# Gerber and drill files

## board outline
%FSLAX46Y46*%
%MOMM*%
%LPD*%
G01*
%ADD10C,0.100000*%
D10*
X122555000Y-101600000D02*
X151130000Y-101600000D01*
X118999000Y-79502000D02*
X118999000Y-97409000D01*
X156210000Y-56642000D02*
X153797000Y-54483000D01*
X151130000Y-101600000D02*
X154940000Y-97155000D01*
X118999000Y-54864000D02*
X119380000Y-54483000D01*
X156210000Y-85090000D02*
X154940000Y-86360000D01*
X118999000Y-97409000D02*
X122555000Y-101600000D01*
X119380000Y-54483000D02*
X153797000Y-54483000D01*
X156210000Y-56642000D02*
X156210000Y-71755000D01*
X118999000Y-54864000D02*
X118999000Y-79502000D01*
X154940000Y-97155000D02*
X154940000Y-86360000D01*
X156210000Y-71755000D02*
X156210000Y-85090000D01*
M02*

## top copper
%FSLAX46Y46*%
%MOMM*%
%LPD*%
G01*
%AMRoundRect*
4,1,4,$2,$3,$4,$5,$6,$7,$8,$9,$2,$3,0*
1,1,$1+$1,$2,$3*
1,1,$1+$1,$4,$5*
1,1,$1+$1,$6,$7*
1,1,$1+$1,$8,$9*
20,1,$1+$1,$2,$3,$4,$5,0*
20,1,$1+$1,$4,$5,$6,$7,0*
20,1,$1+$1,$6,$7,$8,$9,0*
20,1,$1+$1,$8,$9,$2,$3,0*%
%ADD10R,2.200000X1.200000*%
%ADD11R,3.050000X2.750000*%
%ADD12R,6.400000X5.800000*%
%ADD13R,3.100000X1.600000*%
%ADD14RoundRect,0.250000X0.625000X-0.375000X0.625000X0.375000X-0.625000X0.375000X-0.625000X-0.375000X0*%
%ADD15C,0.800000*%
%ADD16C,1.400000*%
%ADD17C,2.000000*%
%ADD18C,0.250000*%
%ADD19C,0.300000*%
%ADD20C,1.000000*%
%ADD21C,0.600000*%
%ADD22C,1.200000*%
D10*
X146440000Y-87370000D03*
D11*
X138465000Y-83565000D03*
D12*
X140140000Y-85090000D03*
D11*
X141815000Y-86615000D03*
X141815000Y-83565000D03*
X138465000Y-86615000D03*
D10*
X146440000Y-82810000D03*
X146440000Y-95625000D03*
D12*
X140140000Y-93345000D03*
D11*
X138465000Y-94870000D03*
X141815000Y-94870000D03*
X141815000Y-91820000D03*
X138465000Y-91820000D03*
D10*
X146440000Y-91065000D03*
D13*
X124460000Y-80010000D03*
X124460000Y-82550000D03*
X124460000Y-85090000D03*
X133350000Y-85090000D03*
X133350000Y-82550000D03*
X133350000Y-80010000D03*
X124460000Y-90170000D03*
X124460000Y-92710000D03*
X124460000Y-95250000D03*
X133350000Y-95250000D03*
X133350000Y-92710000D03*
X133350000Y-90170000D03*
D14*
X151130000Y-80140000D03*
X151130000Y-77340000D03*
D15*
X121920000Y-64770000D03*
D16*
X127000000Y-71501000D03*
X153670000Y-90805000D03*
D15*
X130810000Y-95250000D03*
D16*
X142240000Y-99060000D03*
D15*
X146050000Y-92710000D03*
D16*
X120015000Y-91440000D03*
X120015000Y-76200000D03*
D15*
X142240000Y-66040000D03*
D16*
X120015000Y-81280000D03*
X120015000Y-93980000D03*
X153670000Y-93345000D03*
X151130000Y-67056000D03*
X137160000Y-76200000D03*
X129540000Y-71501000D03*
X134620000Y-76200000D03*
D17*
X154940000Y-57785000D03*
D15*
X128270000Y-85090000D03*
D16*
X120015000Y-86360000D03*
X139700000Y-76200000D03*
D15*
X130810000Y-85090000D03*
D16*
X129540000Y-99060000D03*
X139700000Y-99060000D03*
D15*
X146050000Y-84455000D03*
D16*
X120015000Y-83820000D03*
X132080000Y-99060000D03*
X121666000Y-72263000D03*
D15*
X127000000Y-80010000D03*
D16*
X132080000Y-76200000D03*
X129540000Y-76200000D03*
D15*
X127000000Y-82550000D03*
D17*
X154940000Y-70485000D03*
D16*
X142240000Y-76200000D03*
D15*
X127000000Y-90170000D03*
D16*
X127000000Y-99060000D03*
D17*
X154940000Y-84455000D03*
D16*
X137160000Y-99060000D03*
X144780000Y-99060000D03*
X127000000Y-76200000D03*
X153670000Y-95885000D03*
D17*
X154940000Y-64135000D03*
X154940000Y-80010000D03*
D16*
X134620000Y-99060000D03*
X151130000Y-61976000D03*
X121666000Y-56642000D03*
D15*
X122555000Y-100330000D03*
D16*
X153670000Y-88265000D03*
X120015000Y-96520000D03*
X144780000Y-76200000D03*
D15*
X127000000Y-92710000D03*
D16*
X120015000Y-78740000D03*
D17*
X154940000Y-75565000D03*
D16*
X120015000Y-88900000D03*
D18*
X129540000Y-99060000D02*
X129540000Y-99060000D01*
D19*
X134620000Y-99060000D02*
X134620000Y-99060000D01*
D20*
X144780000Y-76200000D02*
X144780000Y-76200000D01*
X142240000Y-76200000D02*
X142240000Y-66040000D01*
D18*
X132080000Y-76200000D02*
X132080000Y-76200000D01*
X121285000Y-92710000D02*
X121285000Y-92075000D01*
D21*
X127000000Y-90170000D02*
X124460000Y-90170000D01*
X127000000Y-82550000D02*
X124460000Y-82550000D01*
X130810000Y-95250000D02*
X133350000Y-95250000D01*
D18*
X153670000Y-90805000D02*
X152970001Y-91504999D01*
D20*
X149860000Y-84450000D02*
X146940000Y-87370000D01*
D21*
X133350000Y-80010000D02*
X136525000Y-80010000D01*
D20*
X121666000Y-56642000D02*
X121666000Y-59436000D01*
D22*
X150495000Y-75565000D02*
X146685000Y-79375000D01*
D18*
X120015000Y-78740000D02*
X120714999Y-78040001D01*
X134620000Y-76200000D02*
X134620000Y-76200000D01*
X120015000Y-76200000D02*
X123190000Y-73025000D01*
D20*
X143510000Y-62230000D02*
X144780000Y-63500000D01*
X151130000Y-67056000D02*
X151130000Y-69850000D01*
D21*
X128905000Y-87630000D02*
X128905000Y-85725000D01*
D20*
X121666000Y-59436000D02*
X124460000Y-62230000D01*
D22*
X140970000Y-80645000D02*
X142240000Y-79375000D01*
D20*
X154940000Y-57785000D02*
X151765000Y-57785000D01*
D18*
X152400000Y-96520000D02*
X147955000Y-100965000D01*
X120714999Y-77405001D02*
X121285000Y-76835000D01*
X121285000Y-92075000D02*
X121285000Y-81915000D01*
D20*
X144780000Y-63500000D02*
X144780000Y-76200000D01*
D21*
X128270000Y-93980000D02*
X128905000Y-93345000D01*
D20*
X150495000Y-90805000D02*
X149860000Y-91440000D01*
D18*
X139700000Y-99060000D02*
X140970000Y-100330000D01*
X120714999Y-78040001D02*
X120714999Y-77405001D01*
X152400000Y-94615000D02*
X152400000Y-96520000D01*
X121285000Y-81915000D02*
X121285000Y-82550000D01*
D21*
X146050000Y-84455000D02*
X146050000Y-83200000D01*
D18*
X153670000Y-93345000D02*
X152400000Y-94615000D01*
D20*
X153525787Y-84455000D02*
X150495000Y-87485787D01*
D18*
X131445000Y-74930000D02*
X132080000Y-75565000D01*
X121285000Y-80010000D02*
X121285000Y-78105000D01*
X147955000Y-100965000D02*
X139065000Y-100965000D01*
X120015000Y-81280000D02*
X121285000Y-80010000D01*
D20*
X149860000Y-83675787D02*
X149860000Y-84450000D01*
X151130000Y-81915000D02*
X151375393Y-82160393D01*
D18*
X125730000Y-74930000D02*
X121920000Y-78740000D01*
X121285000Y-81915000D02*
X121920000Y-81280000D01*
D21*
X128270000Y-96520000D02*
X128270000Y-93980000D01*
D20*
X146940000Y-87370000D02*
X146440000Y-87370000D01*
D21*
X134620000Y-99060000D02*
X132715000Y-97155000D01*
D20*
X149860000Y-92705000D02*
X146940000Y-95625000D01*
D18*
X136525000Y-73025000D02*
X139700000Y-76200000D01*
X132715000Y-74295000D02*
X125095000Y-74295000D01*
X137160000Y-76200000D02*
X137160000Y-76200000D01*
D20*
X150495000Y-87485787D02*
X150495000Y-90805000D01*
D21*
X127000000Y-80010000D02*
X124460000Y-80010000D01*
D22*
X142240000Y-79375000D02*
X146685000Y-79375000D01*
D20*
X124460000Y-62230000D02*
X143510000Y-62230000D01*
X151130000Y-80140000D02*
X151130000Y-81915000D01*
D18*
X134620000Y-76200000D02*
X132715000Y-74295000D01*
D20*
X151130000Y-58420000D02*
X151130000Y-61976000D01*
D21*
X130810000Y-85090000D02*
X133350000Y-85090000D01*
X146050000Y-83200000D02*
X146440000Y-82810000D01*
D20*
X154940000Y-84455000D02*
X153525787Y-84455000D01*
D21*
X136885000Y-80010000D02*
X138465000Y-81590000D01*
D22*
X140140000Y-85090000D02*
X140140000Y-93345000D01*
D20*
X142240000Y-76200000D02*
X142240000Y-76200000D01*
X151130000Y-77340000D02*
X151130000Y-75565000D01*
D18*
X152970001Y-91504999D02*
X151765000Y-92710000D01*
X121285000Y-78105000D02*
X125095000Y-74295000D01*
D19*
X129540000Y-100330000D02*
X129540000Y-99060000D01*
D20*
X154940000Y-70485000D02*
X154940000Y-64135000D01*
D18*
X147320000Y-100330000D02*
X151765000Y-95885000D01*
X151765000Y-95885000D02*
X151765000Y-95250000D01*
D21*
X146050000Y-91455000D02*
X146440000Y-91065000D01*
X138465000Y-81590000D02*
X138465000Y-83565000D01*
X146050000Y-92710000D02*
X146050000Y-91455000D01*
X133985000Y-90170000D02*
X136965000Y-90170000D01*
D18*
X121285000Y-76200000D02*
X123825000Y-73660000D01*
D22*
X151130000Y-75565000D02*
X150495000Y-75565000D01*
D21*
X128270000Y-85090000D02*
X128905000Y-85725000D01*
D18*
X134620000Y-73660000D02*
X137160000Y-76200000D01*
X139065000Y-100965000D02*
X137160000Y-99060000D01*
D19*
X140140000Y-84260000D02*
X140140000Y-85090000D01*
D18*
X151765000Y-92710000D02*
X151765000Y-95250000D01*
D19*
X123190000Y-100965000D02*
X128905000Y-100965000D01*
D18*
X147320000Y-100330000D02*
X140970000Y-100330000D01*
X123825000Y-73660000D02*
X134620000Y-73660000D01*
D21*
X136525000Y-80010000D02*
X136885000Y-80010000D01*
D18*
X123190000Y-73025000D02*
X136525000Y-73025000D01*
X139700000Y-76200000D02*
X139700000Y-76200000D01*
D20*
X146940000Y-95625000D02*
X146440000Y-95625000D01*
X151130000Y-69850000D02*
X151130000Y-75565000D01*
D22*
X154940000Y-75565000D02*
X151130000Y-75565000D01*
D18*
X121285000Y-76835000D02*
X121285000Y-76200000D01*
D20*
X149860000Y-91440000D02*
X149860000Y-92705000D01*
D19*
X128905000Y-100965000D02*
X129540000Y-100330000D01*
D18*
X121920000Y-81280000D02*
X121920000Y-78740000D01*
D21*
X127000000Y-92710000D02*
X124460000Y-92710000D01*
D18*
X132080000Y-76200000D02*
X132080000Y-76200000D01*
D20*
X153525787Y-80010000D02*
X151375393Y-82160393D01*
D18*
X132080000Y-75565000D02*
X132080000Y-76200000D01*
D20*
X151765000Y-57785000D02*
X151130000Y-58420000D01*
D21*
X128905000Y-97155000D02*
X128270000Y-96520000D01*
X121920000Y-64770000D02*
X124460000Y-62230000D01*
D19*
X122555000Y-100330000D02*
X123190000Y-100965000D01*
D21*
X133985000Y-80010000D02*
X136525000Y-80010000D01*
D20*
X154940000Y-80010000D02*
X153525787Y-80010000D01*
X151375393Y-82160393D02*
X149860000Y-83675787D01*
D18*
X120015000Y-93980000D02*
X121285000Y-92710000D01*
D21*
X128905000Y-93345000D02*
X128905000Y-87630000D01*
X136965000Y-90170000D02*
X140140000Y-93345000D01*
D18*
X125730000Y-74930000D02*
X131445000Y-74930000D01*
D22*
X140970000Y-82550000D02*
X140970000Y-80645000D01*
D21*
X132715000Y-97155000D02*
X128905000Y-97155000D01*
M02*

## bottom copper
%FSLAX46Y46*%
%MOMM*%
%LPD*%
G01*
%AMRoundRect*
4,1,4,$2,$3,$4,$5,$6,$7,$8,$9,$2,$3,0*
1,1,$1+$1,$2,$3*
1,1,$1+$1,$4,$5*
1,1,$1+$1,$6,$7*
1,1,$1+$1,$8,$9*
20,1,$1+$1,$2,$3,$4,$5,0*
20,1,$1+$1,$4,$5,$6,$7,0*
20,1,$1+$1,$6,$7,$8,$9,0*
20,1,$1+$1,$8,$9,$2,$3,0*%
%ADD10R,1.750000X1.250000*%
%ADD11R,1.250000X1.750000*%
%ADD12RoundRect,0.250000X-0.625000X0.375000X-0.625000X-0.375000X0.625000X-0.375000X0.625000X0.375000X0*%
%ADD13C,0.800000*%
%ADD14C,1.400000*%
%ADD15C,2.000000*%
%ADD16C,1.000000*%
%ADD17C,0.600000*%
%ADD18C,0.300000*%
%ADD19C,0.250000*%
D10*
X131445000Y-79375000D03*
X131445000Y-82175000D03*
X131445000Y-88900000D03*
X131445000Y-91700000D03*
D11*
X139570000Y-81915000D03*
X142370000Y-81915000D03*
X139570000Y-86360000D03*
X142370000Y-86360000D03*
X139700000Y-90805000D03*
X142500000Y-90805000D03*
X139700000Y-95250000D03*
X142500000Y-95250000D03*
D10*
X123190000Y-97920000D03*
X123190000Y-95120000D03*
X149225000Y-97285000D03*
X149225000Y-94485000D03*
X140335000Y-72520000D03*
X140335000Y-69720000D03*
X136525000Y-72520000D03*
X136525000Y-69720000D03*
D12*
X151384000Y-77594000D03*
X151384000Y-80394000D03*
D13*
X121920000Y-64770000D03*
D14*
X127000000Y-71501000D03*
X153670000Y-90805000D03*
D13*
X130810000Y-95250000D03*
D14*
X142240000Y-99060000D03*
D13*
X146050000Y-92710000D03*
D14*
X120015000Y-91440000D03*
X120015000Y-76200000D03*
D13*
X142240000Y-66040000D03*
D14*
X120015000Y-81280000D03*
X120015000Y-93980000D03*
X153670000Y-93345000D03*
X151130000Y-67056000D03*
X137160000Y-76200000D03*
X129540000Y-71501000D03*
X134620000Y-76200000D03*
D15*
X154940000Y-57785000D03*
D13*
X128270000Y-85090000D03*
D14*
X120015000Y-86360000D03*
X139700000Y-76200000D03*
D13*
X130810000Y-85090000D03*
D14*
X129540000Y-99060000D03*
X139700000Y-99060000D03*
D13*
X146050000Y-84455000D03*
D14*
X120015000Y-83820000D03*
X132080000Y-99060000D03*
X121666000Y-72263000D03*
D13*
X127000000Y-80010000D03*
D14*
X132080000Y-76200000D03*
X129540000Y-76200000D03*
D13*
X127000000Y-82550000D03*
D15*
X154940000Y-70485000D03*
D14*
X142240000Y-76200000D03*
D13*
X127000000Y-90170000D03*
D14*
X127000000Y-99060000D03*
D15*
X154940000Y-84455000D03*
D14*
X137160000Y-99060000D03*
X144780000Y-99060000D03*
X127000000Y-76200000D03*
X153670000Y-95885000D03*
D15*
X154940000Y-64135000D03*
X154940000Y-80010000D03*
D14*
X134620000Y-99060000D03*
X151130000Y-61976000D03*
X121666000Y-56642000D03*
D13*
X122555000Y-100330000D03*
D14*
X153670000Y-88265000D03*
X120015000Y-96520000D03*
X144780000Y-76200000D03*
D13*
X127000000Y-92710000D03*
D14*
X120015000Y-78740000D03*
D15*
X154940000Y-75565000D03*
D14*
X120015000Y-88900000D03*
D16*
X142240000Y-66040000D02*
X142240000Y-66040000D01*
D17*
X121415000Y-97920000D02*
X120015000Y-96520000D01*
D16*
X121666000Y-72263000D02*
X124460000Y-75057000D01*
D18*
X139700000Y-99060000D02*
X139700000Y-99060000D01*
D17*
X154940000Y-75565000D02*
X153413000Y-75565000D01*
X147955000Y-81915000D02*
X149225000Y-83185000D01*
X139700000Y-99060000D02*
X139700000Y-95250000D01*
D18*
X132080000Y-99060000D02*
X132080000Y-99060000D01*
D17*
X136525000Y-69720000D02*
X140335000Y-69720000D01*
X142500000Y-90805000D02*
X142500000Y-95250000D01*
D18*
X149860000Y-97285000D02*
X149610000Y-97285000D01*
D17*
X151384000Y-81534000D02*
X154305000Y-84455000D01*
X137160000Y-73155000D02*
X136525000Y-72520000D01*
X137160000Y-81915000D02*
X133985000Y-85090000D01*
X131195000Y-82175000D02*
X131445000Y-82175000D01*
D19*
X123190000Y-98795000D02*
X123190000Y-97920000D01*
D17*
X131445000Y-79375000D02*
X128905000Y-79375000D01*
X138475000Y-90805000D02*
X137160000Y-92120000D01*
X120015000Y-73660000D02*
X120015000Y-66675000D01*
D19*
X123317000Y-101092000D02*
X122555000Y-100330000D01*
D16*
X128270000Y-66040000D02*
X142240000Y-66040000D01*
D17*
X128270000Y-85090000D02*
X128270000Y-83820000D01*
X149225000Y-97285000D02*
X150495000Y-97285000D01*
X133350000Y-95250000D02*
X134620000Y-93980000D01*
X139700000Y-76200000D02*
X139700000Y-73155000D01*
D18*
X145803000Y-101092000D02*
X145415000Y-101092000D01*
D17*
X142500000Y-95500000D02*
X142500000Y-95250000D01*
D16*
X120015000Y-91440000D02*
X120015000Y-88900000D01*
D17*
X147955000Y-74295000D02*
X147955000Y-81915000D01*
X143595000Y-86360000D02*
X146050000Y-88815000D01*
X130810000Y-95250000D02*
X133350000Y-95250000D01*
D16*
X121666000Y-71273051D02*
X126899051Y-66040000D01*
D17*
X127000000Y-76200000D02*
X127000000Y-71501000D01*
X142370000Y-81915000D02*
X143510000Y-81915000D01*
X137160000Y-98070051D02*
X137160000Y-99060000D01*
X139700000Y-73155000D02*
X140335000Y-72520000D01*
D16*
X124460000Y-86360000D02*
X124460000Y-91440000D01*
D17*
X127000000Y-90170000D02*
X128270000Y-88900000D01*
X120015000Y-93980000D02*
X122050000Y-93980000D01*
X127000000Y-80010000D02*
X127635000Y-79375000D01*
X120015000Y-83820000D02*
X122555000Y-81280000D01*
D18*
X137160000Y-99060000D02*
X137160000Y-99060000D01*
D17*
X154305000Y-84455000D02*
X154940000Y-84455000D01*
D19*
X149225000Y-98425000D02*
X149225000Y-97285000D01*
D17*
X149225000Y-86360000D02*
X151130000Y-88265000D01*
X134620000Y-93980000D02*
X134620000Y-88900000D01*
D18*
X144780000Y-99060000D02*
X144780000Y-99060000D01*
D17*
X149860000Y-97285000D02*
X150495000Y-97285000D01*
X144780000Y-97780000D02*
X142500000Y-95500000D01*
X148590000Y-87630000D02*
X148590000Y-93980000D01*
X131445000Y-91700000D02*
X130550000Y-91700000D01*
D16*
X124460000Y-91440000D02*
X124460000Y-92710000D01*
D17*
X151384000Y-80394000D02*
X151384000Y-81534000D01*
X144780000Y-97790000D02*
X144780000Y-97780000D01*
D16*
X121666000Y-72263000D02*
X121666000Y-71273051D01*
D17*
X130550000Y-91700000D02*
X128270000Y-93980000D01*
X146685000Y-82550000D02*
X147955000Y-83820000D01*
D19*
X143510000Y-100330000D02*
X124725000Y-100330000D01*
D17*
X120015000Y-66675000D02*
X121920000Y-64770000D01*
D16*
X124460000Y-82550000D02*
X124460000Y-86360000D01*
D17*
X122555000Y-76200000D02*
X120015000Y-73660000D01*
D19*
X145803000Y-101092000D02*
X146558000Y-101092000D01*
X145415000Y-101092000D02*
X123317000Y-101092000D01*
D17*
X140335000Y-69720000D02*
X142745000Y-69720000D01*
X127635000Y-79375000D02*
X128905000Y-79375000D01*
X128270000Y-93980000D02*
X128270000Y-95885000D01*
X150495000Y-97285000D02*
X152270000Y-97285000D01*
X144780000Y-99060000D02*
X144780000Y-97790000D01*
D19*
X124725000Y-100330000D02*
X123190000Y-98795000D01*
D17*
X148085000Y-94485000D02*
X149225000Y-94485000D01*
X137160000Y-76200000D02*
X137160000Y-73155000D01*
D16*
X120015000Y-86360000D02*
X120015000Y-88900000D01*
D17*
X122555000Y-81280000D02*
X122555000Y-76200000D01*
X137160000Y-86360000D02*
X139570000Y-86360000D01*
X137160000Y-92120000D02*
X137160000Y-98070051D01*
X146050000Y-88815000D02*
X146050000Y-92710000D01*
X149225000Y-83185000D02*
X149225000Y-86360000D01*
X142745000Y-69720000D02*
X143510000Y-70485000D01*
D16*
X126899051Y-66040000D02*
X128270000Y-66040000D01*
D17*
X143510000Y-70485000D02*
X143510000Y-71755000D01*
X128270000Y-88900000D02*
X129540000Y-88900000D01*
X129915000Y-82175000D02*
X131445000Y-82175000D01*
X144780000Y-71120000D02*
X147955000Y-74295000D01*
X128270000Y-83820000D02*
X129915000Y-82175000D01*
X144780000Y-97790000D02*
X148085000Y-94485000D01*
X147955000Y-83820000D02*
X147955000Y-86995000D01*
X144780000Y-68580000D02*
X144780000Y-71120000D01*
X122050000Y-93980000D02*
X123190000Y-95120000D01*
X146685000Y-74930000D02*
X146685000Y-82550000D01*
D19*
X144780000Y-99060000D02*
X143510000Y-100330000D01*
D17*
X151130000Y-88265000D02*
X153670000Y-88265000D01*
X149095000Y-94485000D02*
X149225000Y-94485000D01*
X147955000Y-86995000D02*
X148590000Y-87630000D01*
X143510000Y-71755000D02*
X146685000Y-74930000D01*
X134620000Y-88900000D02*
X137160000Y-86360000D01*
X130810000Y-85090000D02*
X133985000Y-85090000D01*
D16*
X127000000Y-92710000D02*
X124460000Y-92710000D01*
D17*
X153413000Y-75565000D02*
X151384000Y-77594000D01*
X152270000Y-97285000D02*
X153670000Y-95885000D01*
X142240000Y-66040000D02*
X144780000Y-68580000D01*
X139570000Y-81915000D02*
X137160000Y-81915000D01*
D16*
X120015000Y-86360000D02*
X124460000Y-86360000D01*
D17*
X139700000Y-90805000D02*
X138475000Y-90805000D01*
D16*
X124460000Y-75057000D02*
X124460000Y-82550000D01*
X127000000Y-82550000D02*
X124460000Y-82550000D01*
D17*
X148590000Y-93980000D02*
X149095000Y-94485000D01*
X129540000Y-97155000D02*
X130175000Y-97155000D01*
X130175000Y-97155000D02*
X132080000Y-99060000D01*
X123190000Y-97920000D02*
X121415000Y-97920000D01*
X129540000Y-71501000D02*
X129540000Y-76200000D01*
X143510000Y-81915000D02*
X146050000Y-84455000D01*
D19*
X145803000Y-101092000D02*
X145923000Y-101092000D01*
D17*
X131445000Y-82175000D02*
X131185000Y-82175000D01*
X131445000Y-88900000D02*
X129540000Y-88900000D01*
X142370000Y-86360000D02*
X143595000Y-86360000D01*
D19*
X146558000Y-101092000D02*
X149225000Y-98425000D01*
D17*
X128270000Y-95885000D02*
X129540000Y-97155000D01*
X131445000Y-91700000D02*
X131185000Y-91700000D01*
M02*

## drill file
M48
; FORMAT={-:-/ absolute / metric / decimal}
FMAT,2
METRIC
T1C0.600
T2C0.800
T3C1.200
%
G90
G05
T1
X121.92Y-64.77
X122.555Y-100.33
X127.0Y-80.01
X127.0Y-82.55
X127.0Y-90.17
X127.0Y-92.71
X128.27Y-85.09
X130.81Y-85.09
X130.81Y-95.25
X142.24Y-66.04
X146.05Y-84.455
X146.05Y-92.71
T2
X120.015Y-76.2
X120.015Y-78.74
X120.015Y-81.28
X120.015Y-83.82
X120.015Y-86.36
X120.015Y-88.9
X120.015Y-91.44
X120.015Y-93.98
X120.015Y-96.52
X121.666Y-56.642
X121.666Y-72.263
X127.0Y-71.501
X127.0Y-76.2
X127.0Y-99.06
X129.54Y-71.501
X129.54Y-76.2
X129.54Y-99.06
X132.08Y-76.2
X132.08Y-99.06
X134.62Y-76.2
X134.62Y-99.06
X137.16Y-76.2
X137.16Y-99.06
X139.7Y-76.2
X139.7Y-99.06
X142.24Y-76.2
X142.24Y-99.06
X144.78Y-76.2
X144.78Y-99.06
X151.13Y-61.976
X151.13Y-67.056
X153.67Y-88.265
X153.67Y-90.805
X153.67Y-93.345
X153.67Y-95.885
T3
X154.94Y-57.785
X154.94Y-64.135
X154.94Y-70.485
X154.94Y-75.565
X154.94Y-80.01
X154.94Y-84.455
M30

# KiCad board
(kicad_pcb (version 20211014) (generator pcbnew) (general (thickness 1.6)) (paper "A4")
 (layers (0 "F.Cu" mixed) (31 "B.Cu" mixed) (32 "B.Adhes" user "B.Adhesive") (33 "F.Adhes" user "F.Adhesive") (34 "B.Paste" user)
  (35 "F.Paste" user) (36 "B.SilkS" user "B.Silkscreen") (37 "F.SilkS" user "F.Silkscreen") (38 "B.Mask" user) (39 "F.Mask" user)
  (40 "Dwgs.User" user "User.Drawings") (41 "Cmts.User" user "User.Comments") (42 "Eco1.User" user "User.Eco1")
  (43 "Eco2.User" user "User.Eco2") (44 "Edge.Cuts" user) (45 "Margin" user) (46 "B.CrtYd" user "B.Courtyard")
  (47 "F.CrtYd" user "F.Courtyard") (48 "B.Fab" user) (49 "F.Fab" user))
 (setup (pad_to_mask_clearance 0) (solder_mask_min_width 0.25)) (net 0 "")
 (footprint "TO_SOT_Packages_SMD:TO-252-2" (layer "F.Cu") (at 142.24 85.09 180)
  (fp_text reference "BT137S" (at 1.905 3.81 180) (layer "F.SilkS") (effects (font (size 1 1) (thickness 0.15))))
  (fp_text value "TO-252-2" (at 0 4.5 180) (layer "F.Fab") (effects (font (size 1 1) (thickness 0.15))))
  (pad "1" smd rect locked (at -4.2 -2.28 180) (size 2.2 1.2) (layers "F.Cu" "F.Paste" "F.Mask"))
  (pad "2" smd rect locked (at 3.775 1.525 180) (size 3.05 2.75) (layers "F.Cu" "F.Paste"))
  (pad "2" smd rect locked (at 2.1 0 180) (size 6.4 5.8) (layers "F.Cu" "F.Mask"))
  (pad "2" smd rect locked (at 0.425 -1.525 180) (size 3.05 2.75) (layers "F.Cu" "F.Paste"))
  (pad "2" smd rect locked (at 0.425 1.525 180) (size 3.05 2.75) (layers "F.Cu" "F.Paste"))
  (pad "2" smd rect locked (at 3.775 -1.525 180) (size 3.05 2.75) (layers "F.Cu" "F.Paste"))
  (pad "3" smd rect locked (at -4.2 2.28 180) (size 2.2 1.2) (layers "F.Cu" "F.Paste" "F.Mask")))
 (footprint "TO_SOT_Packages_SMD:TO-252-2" (layer "F.Cu") (at 142.24 93.345 180)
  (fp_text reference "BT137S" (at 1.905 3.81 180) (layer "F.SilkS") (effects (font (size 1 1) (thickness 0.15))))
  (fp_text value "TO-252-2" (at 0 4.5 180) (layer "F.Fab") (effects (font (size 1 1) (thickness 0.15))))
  (pad "1" smd rect locked (at -4.2 -2.28 180) (size 2.2 1.2) (layers "F.Cu" "F.Paste" "F.Mask"))
  (pad "2" smd rect locked (at 2.1 0 180) (size 6.4 5.8) (layers "F.Cu" "F.Mask"))
  (pad "2" smd rect locked (at 3.775 -1.525 180) (size 3.05 2.75) (layers "F.Cu" "F.Paste"))
  (pad "2" smd rect locked (at 0.425 -1.525 180) (size 3.05 2.75) (layers "F.Cu" "F.Paste"))
  (pad "2" smd rect locked (at 0.425 1.525 180) (size 3.05 2.75) (layers "F.Cu" "F.Paste"))
  (pad "2" smd rect locked (at 3.775 1.525 180) (size 3.05 2.75) (layers "F.Cu" "F.Paste"))
  (pad "3" smd rect locked (at -4.2 2.28 180) (size 2.2 1.2) (layers "F.Cu" "F.Paste" "F.Mask")))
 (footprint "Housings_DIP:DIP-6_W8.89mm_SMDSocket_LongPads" (layer "F.Cu") (at 128.905 82.55)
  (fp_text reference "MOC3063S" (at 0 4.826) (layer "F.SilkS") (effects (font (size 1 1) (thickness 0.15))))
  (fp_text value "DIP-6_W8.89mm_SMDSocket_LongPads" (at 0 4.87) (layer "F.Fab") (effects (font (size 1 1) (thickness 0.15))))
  (pad "1" smd rect locked (at -4.445 -2.54) (size 3.1 1.6) (layers "F.Cu" "F.Paste" "F.Mask"))
  (pad "2" smd rect locked (at -4.445 0) (size 3.1 1.6) (layers "F.Cu" "F.Paste" "F.Mask"))
  (pad "3" smd rect locked (at -4.445 2.54) (size 3.1 1.6) (layers "F.Cu" "F.Paste" "F.Mask"))
  (pad "4" smd rect locked (at 4.445 2.54) (size 3.1 1.6) (layers "F.Cu" "F.Paste" "F.Mask"))
  (pad "5" smd rect locked (at 4.445 0) (size 3.1 1.6) (layers "F.Cu" "F.Paste" "F.Mask"))
  (pad "6" smd rect locked (at 4.445 -2.54) (size 3.1 1.6) (layers "F.Cu" "F.Paste" "F.Mask")))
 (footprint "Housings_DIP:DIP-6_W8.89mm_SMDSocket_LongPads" (layer "F.Cu") (at 128.905 92.71)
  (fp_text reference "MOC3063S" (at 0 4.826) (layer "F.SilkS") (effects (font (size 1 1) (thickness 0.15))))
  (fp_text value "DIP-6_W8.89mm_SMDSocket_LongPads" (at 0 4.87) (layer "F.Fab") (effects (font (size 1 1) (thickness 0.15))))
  (pad "1" smd rect locked (at -4.445 -2.54) (size 3.1 1.6) (layers "F.Cu" "F.Paste" "F.Mask"))
  (pad "2" smd rect locked (at -4.445 0) (size 3.1 1.6) (layers "F.Cu" "F.Paste" "F.Mask"))
  (pad "3" smd rect locked (at -4.445 2.54) (size 3.1 1.6) (layers "F.Cu" "F.Paste" "F.Mask"))
  (pad "4" smd rect locked (at 4.445 2.54) (size 3.1 1.6) (layers "F.Cu" "F.Paste" "F.Mask"))
  (pad "5" smd rect locked (at 4.445 0) (size 3.1 1.6) (layers "F.Cu" "F.Paste" "F.Mask"))
  (pad "6" smd rect locked (at 4.445 -2.54) (size 3.1 1.6) (layers "F.Cu" "F.Paste" "F.Mask")))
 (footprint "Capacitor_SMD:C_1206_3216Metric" (layer "F.Cu") (at 151.13 78.74 90)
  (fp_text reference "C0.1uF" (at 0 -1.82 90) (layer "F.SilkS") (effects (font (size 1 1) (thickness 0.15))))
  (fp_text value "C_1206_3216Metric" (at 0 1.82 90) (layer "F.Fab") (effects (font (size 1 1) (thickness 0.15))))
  (pad "1" smd roundrect locked (at -1.4 0 90) (size 1.25 1.75) (layers "F.Cu" "F.Paste" "F.Mask") (roundrect_rratio 0.2))
  (pad "2" smd roundrect locked (at 1.4 0 90) (size 1.25 1.75) (layers "F.Cu" "F.Paste" "F.Mask") (roundrect_rratio 0.2)))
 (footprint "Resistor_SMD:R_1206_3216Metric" (layer "B.Cu") (at 131.445 80.775 -90)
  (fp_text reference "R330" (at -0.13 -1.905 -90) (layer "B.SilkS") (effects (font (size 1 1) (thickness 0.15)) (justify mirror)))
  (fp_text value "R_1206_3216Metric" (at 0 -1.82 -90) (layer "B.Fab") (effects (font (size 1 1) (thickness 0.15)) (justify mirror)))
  (pad "1" smd rect locked (at -1.4 0 270) (size 1.25 1.75) (layers "B.Cu" "B.Paste" "B.Mask"))
  (pad "2" smd rect locked (at 1.4 0 270) (size 1.25 1.75) (layers "B.Cu" "B.Paste" "B.Mask")))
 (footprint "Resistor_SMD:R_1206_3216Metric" (layer "B.Cu") (at 131.445 90.3 -90)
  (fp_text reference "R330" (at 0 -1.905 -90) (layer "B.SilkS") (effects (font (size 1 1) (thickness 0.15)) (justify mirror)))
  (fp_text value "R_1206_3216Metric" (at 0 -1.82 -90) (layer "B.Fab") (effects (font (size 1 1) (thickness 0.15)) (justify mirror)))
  (pad "1" smd rect locked (at -1.4 0 270) (size 1.25 1.75) (layers "B.Cu" "B.Paste" "B.Mask"))
  (pad "2" smd rect locked (at 1.4 0 270) (size 1.25 1.75) (layers "B.Cu" "B.Paste" "B.Mask")))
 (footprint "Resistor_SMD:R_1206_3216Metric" (layer "B.Cu") (at 140.97 81.915)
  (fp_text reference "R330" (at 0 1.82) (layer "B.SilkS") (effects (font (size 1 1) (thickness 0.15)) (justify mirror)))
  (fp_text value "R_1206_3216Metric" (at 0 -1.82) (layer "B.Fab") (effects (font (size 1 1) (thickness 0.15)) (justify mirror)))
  (pad "1" smd rect locked (at -1.4 0) (size 1.25 1.75) (layers "B.Cu" "B.Paste" "B.Mask"))
  (pad "2" smd rect locked (at 1.4 0) (size 1.25 1.75) (layers "B.Cu" "B.Paste" "B.Mask")))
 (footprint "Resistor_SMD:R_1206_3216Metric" (layer "B.Cu") (at 140.97 86.36)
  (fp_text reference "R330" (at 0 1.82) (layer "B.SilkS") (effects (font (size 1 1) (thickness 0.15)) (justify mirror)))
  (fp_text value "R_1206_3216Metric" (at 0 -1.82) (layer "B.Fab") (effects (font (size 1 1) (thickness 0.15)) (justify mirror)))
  (pad "1" smd rect locked (at -1.4 0) (size 1.25 1.75) (layers "B.Cu" "B.Paste" "B.Mask"))
  (pad "2" smd rect locked (at 1.4 0) (size 1.25 1.75) (layers "B.Cu" "B.Paste" "B.Mask")))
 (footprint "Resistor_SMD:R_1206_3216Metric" (layer "B.Cu") (at 141.1 90.805)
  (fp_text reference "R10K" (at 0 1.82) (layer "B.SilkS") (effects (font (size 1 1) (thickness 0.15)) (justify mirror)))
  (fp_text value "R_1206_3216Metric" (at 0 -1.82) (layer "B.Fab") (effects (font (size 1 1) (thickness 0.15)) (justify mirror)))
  (pad "1" smd rect locked (at -1.4 0) (size 1.25 1.75) (layers "B.Cu" "B.Paste" "B.Mask"))
  (pad "2" smd rect locked (at 1.4 0) (size 1.25 1.75) (layers "B.Cu" "B.Paste" "B.Mask")))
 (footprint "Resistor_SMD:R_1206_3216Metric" (layer "B.Cu") (at 141.1 95.25)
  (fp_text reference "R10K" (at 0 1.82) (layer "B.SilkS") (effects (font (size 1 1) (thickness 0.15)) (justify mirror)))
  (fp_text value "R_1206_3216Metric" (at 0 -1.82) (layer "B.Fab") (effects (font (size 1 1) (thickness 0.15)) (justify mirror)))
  (pad "1" smd rect locked (at -1.4 0) (size 1.25 1.75) (layers "B.Cu" "B.Paste" "B.Mask"))
  (pad "2" smd rect locked (at 1.4 0) (size 1.25 1.75) (layers "B.Cu" "B.Paste" "B.Mask")))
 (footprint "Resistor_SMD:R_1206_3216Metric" (layer "B.Cu") (at 123.19 96.52 90)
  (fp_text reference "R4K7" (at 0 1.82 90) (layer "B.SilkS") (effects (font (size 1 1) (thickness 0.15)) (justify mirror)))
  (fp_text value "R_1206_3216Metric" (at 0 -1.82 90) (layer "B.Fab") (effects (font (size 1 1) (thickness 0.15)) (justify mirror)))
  (pad "1" smd rect locked (at -1.4 0 90) (size 1.25 1.75) (layers "B.Cu" "B.Paste" "B.Mask"))
  (pad "2" smd rect locked (at 1.4 0 90) (size 1.25 1.75) (layers "B.Cu" "B.Paste" "B.Mask")))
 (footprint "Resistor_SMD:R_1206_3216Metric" (layer "B.Cu") (at 149.225 95.885 90)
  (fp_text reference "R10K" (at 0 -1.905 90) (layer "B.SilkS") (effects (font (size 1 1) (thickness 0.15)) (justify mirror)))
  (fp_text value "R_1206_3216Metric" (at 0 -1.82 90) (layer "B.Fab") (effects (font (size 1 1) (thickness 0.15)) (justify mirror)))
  (pad "1" smd rect locked (at -1.4 0 90) (size 1.25 1.75) (layers "B.Cu" "B.Paste" "B.Mask"))
  (pad "2" smd rect locked (at 1.4 0 90) (size 1.25 1.75) (layers "B.Cu" "B.Paste" "B.Mask")))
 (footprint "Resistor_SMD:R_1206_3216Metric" (layer "B.Cu") (at 140.335 71.12 90)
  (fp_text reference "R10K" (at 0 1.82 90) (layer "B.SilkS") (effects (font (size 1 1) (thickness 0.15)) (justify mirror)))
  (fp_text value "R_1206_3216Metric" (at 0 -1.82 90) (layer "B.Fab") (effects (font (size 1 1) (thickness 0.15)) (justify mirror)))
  (pad "1" smd rect locked (at -1.4 0 90) (size 1.25 1.75) (layers "B.Cu" "B.Paste" "B.Mask"))
  (pad "2" smd rect locked (at 1.4 0 90) (size 1.25 1.75) (layers "B.Cu" "B.Paste" "B.Mask")))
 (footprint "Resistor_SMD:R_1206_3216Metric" (layer "B.Cu") (at 136.525 71.12 90)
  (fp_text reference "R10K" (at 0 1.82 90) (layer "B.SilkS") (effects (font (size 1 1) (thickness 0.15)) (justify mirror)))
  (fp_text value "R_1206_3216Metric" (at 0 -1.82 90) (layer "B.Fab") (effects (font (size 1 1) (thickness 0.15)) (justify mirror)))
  (pad "1" smd rect locked (at -1.4 0 90) (size 1.25 1.75) (layers "B.Cu" "B.Paste" "B.Mask"))
  (pad "2" smd rect locked (at 1.4 0 90) (size 1.25 1.75) (layers "B.Cu" "B.Paste" "B.Mask")))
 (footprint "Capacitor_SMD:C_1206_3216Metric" (layer "B.Cu") (at 151.384 78.994 -90)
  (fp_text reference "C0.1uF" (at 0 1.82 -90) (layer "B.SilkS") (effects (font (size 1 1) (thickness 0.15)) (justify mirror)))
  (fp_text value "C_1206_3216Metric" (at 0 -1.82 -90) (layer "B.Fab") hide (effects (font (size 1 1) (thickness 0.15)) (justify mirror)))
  (pad "1" smd roundrect locked (at -1.4 0 270) (size 1.25 1.75) (layers "B.Cu" "B.Paste" "B.Mask") (roundrect_rratio 0.2))
  (pad "2" smd roundrect locked (at 1.4 0 270) (size 1.25 1.75) (layers "B.Cu" "B.Paste" "B.Mask") (roundrect_rratio 0.2)))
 (gr_line (start 122.555 101.6) (end 151.13 101.6) (layer "Edge.Cuts") (width 0.1))
 (gr_line (start 118.999 79.502) (end 118.999 97.409) (layer "Edge.Cuts") (width 0.1))
 (gr_line (start 156.21 56.642) (end 153.797 54.483) (layer "Edge.Cuts") (width 0.1))
 (gr_line (start 151.13 101.6) (end 154.94 97.155) (layer "Edge.Cuts") (width 0.1))
 (gr_line (start 118.999 54.864) (end 119.38 54.483) (layer "Edge.Cuts") (width 0.1))
 (gr_line (start 156.21 85.09) (end 154.94 86.36) (layer "Edge.Cuts") (width 0.1))
 (gr_line (start 118.999 97.409) (end 122.555 101.6) (layer "Edge.Cuts") (width 0.1))
 (gr_line (start 119.38 54.483) (end 153.797 54.483) (layer "Edge.Cuts") (width 0.1))
 (gr_line (start 156.21 56.642) (end 156.21 71.755) (layer "Edge.Cuts") (width 0.1))
 (gr_line (start 118.999 54.864) (end 118.999 79.502) (layer "Edge.Cuts") (width 0.1))
 (gr_line (start 154.94 97.155) (end 154.94 86.36) (layer "Edge.Cuts") (width 0.1))
 (gr_line (start 156.21 71.755) (end 156.21 85.09) (layer "Edge.Cuts") (width 0.1))
 (segment (start 129.54 99.06) (end 129.54 99.06) (width 0.25) (layer "F.Cu") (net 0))
 (segment (start 134.62 99.06) (end 134.62 99.06) (width 0.3) (layer "F.Cu") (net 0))
 (segment (start 144.78 76.2) (end 144.78 76.2) (width 1) (layer "F.Cu") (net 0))
 (segment (start 142.24 76.2) (end 142.24 66.04) (width 1) (layer "F.Cu") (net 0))
 (segment (start 132.08 76.2) (end 132.08 76.2) (width 0.25) (layer "F.Cu") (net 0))
 (segment (start 121.285 92.71) (end 121.285 92.075) (width 0.25) (layer "F.Cu") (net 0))
 (segment (start 127 90.17) (end 124.46 90.17) (width 0.6) (layer "F.Cu") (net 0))
 (segment (start 127 82.55) (end 124.46 82.55) (width 0.6) (layer "F.Cu") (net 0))
 (segment (start 130.81 95.25) (end 133.35 95.25) (width 0.6) (layer "F.Cu") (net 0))
 (segment (start 153.67 90.805) (end 152.970001 91.504999) (width 0.25) (layer "F.Cu") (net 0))
 (segment (start 149.86 84.45) (end 146.94 87.37) (width 1) (layer "F.Cu") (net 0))
 (segment (start 133.35 80.01) (end 136.525 80.01) (width 0.6) (layer "F.Cu") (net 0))
 (segment (start 121.666 56.642) (end 121.666 59.436) (width 1) (layer "F.Cu") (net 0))
 (segment (start 150.495 75.565) (end 146.685 79.375) (width 1.2) (layer "F.Cu") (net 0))
 (segment (start 120.015 78.74) (end 120.714999 78.040001) (width 0.25) (layer "F.Cu") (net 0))
 (segment (start 134.62 76.2) (end 134.62 76.2) (width 0.25) (layer "F.Cu") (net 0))
 (segment (start 120.015 76.2) (end 123.19 73.025) (width 0.25) (layer "F.Cu") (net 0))
 (segment (start 143.51 62.23) (end 144.78 63.5) (width 1) (layer "F.Cu") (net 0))
 (segment (start 151.13 67.056) (end 151.13 69.85) (width 1) (layer "F.Cu") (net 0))
 (segment (start 128.905 87.63) (end 128.905 85.725) (width 0.6) (layer "F.Cu") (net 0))
 (segment (start 121.666 59.436) (end 124.46 62.23) (width 1) (layer "F.Cu") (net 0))
 (segment (start 140.97 80.645) (end 142.24 79.375) (width 1.2) (layer "F.Cu") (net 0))
 (segment (start 154.94 57.785) (end 151.765 57.785) (width 1) (layer "F.Cu") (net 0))
 (segment (start 152.4 96.52) (end 147.955 100.965) (width 0.25) (layer "F.Cu") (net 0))
 (segment (start 120.714999 77.405001) (end 121.285 76.835) (width 0.25) (layer "F.Cu") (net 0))
 (segment (start 121.285 92.075) (end 121.285 81.915) (width 0.25) (layer "F.Cu") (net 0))
 (segment (start 144.78 63.5) (end 144.78 76.2) (width 1) (layer "F.Cu") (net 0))
 (segment (start 128.27 93.98) (end 128.905 93.345) (width 0.6) (layer "F.Cu") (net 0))
 (segment (start 150.495 90.805) (end 149.86 91.44) (width 1) (layer "F.Cu") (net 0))
 (segment (start 139.7 99.06) (end 140.97 100.33) (width 0.25) (layer "F.Cu") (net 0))
 (segment (start 120.714999 78.040001) (end 120.714999 77.405001) (width 0.25) (layer "F.Cu") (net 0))
 (segment (start 152.4 94.615) (end 152.4 96.52) (width 0.25) (layer "F.Cu") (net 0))
 (segment (start 121.285 81.915) (end 121.285 82.55) (width 0.25) (layer "F.Cu") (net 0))
 (segment (start 146.05 84.455) (end 146.05 83.2) (width 0.6) (layer "F.Cu") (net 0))
 (segment (start 153.67 93.345) (end 152.4 94.615) (width 0.25) (layer "F.Cu") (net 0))
 (segment (start 153.525787 84.455) (end 150.495 87.485787) (width 1) (layer "F.Cu") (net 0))
 (segment (start 131.445 74.93) (end 132.08 75.565) (width 0.25) (layer "F.Cu") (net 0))
 (segment (start 121.285 80.01) (end 121.285 78.105) (width 0.25) (layer "F.Cu") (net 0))
 (segment (start 147.955 100.965) (end 139.065 100.965) (width 0.25) (layer "F.Cu") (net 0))
 (segment (start 120.015 81.28) (end 121.285 80.01) (width 0.25) (layer "F.Cu") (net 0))
 (segment (start 149.86 83.675787) (end 149.86 84.45) (width 1) (layer "F.Cu") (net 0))
 (segment (start 151.13 81.915) (end 151.375393 82.160393) (width 1) (layer "F.Cu") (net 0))
 (segment (start 125.73 74.93) (end 121.92 78.74) (width 0.25) (layer "F.Cu") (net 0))
 (segment (start 121.285 81.915) (end 121.92 81.28) (width 0.25) (layer "F.Cu") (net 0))
 (segment (start 128.27 96.52) (end 128.27 93.98) (width 0.6) (layer "F.Cu") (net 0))
 (segment (start 146.94 87.37) (end 146.44 87.37) (width 1) (layer "F.Cu") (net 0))
 (segment (start 134.62 99.06) (end 132.715 97.155) (width 0.6) (layer "F.Cu") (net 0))
 (segment (start 149.86 92.705) (end 146.94 95.625) (width 1) (layer "F.Cu") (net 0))
 (segment (start 136.525 73.025) (end 139.7 76.2) (width 0.25) (layer "F.Cu") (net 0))
 (segment (start 132.715 74.295) (end 125.095 74.295) (width 0.25) (layer "F.Cu") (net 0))
 (segment (start 137.16 76.2) (end 137.16 76.2) (width 0.25) (layer "F.Cu") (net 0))
 (segment (start 150.495 87.485787) (end 150.495 90.805) (width 1) (layer "F.Cu") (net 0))
 (segment (start 127 80.01) (end 124.46 80.01) (width 0.6) (layer "F.Cu") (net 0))
 (segment (start 142.24 79.375) (end 146.685 79.375) (width 1.2) (layer "F.Cu") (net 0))
 (segment (start 124.46 62.23) (end 143.51 62.23) (width 1) (layer "F.Cu") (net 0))
 (segment (start 151.13 80.14) (end 151.13 81.915) (width 1) (layer "F.Cu") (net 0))
 (segment (start 134.62 76.2) (end 132.715 74.295) (width 0.25) (layer "F.Cu") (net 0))
 (segment (start 151.13 58.42) (end 151.13 61.976) (width 1) (layer "F.Cu") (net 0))
 (segment (start 130.81 85.09) (end 133.35 85.09) (width 0.6) (layer "F.Cu") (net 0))
 (segment (start 146.05 83.2) (end 146.44 82.81) (width 0.6) (layer "F.Cu") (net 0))
 (segment (start 154.94 84.455) (end 153.525787 84.455) (width 1) (layer "F.Cu") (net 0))
 (segment (start 136.885 80.01) (end 138.465 81.59) (width 0.6) (layer "F.Cu") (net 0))
 (segment (start 140.14 85.09) (end 140.14 93.345) (width 1.2) (layer "F.Cu") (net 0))
 (segment (start 142.24 76.2) (end 142.24 76.2) (width 1) (layer "F.Cu") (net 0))
 (segment (start 151.13 77.34) (end 151.13 75.565) (width 1) (layer "F.Cu") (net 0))
 (segment (start 152.970001 91.504999) (end 151.765 92.71) (width 0.25) (layer "F.Cu") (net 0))
 (segment (start 121.285 78.105) (end 125.095 74.295) (width 0.25) (layer "F.Cu") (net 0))
 (segment (start 129.54 100.33) (end 129.54 99.06) (width 0.3) (layer "F.Cu") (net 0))
 (segment (start 154.94 70.485) (end 154.94 64.135) (width 1) (layer "F.Cu") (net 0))
 (segment (start 147.32 100.33) (end 151.765 95.885) (width 0.25) (layer "F.Cu") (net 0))
 (segment (start 151.765 95.885) (end 151.765 95.25) (width 0.25) (layer "F.Cu") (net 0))
 (segment (start 146.05 91.455) (end 146.44 91.065) (width 0.6) (layer "F.Cu") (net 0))
 (segment (start 138.465 81.59) (end 138.465 83.565) (width 0.6) (layer "F.Cu") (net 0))
 (segment (start 146.05 92.71) (end 146.05 91.455) (width 0.6) (layer "F.Cu") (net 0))
 (segment (start 133.985 90.17) (end 136.965 90.17) (width 0.6) (layer "F.Cu") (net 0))
 (segment (start 121.285 76.2) (end 123.825 73.66) (width 0.25) (layer "F.Cu") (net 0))
 (segment (start 151.13 75.565) (end 150.495 75.565) (width 1.2) (layer "F.Cu") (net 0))
 (segment (start 128.27 85.09) (end 128.905 85.725) (width 0.6) (layer "F.Cu") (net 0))
 (segment (start 134.62 73.66) (end 137.16 76.2) (width 0.25) (layer "F.Cu") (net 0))
 (segment (start 139.065 100.965) (end 137.16 99.06) (width 0.25) (layer "F.Cu") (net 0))
 (segment (start 140.14 84.26) (end 140.14 85.09) (width 0.3) (layer "F.Cu") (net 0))
 (segment (start 151.765 92.71) (end 151.765 95.25) (width 0.25) (layer "F.Cu") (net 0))
 (segment (start 123.19 100.965) (end 128.905 100.965) (width 0.3) (layer "F.Cu") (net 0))
 (segment (start 147.32 100.33) (end 140.97 100.33) (width 0.25) (layer "F.Cu") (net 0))
 (segment (start 123.825 73.66) (end 134.62 73.66) (width 0.25) (layer "F.Cu") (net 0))
 (segment (start 136.525 80.01) (end 136.885 80.01) (width 0.6) (layer "F.Cu") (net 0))
 (segment (start 123.19 73.025) (end 136.525 73.025) (width 0.25) (layer "F.Cu") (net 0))
 (segment (start 139.7 76.2) (end 139.7 76.2) (width 0.25) (layer "F.Cu") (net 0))
 (segment (start 146.94 95.625) (end 146.44 95.625) (width 1) (layer "F.Cu") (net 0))
 (segment (start 151.13 69.85) (end 151.13 75.565) (width 1) (layer "F.Cu") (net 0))
 (segment (start 154.94 75.565) (end 151.13 75.565) (width 1.2) (layer "F.Cu") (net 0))
 (segment (start 121.285 76.835) (end 121.285 76.2) (width 0.25) (layer "F.Cu") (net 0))
 (segment (start 149.86 91.44) (end 149.86 92.705) (width 1) (layer "F.Cu") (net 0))
 (segment (start 128.905 100.965) (end 129.54 100.33) (width 0.3) (layer "F.Cu") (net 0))
 (segment (start 121.92 81.28) (end 121.92 78.74) (width 0.25) (layer "F.Cu") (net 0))
 (segment (start 127 92.71) (end 124.46 92.71) (width 0.6) (layer "F.Cu") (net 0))
 (segment (start 132.08 76.2) (end 132.08 76.2) (width 0.25) (layer "F.Cu") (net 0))
 (segment (start 153.525787 80.01) (end 151.375393 82.160393) (width 1) (layer "F.Cu") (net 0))
 (segment (start 132.08 75.565) (end 132.08 76.2) (width 0.25) (layer "F.Cu") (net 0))
 (segment (start 151.765 57.785) (end 151.13 58.42) (width 1) (layer "F.Cu") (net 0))
 (segment (start 128.905 97.155) (end 128.27 96.52) (width 0.6) (layer "F.Cu") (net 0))
 (segment (start 121.92 64.77) (end 124.46 62.23) (width 0.6) (layer "F.Cu") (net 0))
 (segment (start 122.555 100.33) (end 123.19 100.965) (width 0.3) (layer "F.Cu") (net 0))
 (segment (start 133.985 80.01) (end 136.525 80.01) (width 0.6) (layer "F.Cu") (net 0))
 (segment (start 154.94 80.01) (end 153.525787 80.01) (width 1) (layer "F.Cu") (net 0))
 (segment (start 151.375393 82.160393) (end 149.86 83.675787) (width 1) (layer "F.Cu") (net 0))
 (segment (start 120.015 93.98) (end 121.285 92.71) (width 0.25) (layer "F.Cu") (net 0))
 (segment (start 128.905 93.345) (end 128.905 87.63) (width 0.6) (layer "F.Cu") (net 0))
 (segment (start 136.965 90.17) (end 140.14 93.345) (width 0.6) (layer "F.Cu") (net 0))
 (segment (start 125.73 74.93) (end 131.445 74.93) (width 0.25) (layer "F.Cu") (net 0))
 (segment (start 140.97 82.55) (end 140.97 80.645) (width 1.2) (layer "F.Cu") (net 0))
 (segment (start 132.715 97.155) (end 128.905 97.155) (width 0.6) (layer "F.Cu") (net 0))
 (via (at 121.92 64.77) (size 0.8) (drill 0.6) (layers "F.Cu" "B.Cu") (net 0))
 (via (at 127 71.501) (size 1.4) (drill 0.8) (layers "F.Cu" "B.Cu") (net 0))
 (via (at 153.67 90.805) (size 1.4) (drill 0.8) (layers "F.Cu" "B.Cu") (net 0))
 (via (at 130.81 95.25) (size 0.8) (drill 0.6) (layers "F.Cu" "B.Cu") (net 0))
 (via (at 142.24 99.06) (size 1.4) (drill 0.8) (layers "F.Cu" "B.Cu") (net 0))
 (via (at 146.05 92.71) (size 0.8) (drill 0.6) (layers "F.Cu" "B.Cu") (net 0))
 (via (at 120.015 91.44) (size 1.4) (drill 0.8) (layers "F.Cu" "B.Cu") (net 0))
 (via (at 120.015 76.2) (size 1.4) (drill 0.8) (layers "F.Cu" "B.Cu") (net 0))
 (via (at 142.24 66.04) (size 0.8) (drill 0.6) (layers "F.Cu" "B.Cu") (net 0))
 (via (at 120.015 81.28) (size 1.4) (drill 0.8) (layers "F.Cu" "B.Cu") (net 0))
 (via (at 120.015 93.98) (size 1.4) (drill 0.8) (layers "F.Cu" "B.Cu") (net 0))
 (via (at 153.67 93.345) (size 1.4) (drill 0.8) (layers "F.Cu" "B.Cu") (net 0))
 (via (at 151.13 67.056) (size 1.4) (drill 0.8) (layers "F.Cu" "B.Cu") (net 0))
 (via (at 137.16 76.2) (size 1.4) (drill 0.8) (layers "F.Cu" "B.Cu") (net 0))
 (via (at 129.54 71.501) (size 1.4) (drill 0.8) (layers "F.Cu" "B.Cu") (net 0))
 (via (at 134.62 76.2) (size 1.4) (drill 0.8) (layers "F.Cu" "B.Cu") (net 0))
 (via (at 154.94 57.785) (size 2) (drill 1.2) (layers "F.Cu" "B.Cu") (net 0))
 (via (at 128.27 85.09) (size 0.8) (drill 0.6) (layers "F.Cu" "B.Cu") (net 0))
 (via (at 120.015 86.36) (size 1.4) (drill 0.8) (layers "F.Cu" "B.Cu") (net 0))
 (via (at 139.7 76.2) (size 1.4) (drill 0.8) (layers "F.Cu" "B.Cu") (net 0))
 (via (at 130.81 85.09) (size 0.8) (drill 0.6) (layers "F.Cu" "B.Cu") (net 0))
 (via (at 129.54 99.06) (size 1.4) (drill 0.8) (layers "F.Cu" "B.Cu") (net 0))
 (via (at 139.7 99.06) (size 1.4) (drill 0.8) (layers "F.Cu" "B.Cu") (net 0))
 (via (at 146.05 84.455) (size 0.8) (drill 0.6) (layers "F.Cu" "B.Cu") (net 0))
 (via (at 120.015 83.82) (size 1.4) (drill 0.8) (layers "F.Cu" "B.Cu") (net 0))
 (via (at 132.08 99.06) (size 1.4) (drill 0.8) (layers "F.Cu" "B.Cu") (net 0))
 (via (at 121.666 72.263) (size 1.4) (drill 0.8) (layers "F.Cu" "B.Cu") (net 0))
 (via (at 127 80.01) (size 0.8) (drill 0.6) (layers "F.Cu" "B.Cu") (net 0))
 (via (at 132.08 76.2) (size 1.4) (drill 0.8) (layers "F.Cu" "B.Cu") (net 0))
 (via (at 129.54 76.2) (size 1.4) (drill 0.8) (layers "F.Cu" "B.Cu") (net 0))
 (via (at 127 82.55) (size 0.8) (drill 0.6) (layers "F.Cu" "B.Cu") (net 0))
 (via (at 154.94 70.485) (size 2) (drill 1.2) (layers "F.Cu" "B.Cu") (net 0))
 (via (at 142.24 76.2) (size 1.4) (drill 0.8) (layers "F.Cu" "B.Cu") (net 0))
 (via (at 127 90.17) (size 0.8) (drill 0.6) (layers "F.Cu" "B.Cu") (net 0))
 (via (at 127 99.06) (size 1.4) (drill 0.8) (layers "F.Cu" "B.Cu") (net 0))
 (via (at 154.94 84.455) (size 2) (drill 1.2) (layers "F.Cu" "B.Cu") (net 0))
 (via (at 137.16 99.06) (size 1.4) (drill 0.8) (layers "F.Cu" "B.Cu") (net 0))
 (via (at 144.78 99.06) (size 1.4) (drill 0.8) (layers "F.Cu" "B.Cu") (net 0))
 (via (at 127 76.2) (size 1.4) (drill 0.8) (layers "F.Cu" "B.Cu") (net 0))
 (via (at 153.67 95.885) (size 1.4) (drill 0.8) (layers "F.Cu" "B.Cu") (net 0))
 (via (at 154.94 64.135) (size 2) (drill 1.2) (layers "F.Cu" "B.Cu") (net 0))
 (via (at 154.94 80.01) (size 2) (drill 1.2) (layers "F.Cu" "B.Cu") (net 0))
 (via (at 134.62 99.06) (size 1.4) (drill 0.8) (layers "F.Cu" "B.Cu") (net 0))
 (via (at 151.13 61.976) (size 1.4) (drill 0.8) (layers "F.Cu" "B.Cu") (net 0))
 (via (at 121.666 56.642) (size 1.4) (drill 0.8) (layers "F.Cu" "B.Cu") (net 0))
 (via (at 122.555 100.33) (size 0.8) (drill 0.6) (layers "F.Cu" "B.Cu") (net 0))
 (via (at 153.67 88.265) (size 1.4) (drill 0.8) (layers "F.Cu" "B.Cu") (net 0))
 (via (at 120.015 96.52) (size 1.4) (drill 0.8) (layers "F.Cu" "B.Cu") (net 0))
 (via (at 144.78 76.2) (size 1.4) (drill 0.8) (layers "F.Cu" "B.Cu") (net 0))
 (via (at 127 92.71) (size 0.8) (drill 0.6) (layers "F.Cu" "B.Cu") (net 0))
 (via (at 120.015 78.74) (size 1.4) (drill 0.8) (layers "F.Cu" "B.Cu") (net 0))
 (via (at 154.94 75.565) (size 2) (drill 1.2) (layers "F.Cu" "B.Cu") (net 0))
 (via (at 120.015 88.9) (size 1.4) (drill 0.8) (layers "F.Cu" "B.Cu") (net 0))
 (segment (start 142.24 66.04) (end 142.24 66.04) (width 1) (layer "B.Cu") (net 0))
 (segment (start 121.415 97.92) (end 120.015 96.52) (width 0.6) (layer "B.Cu") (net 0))
 (segment (start 121.666 72.263) (end 124.46 75.057) (width 1) (layer "B.Cu") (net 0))
 (segment (start 139.7 99.06) (end 139.7 99.06) (width 0.3) (layer "B.Cu") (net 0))
 (segment (start 154.94 75.565) (end 153.413 75.565) (width 0.6) (layer "B.Cu") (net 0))
 (segment (start 147.955 81.915) (end 149.225 83.185) (width 0.6) (layer "B.Cu") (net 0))
 (segment (start 139.7 99.06) (end 139.7 95.25) (width 0.6) (layer "B.Cu") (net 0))
 (segment (start 132.08 99.06) (end 132.08 99.06) (width 0.3) (layer "B.Cu") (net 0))
 (segment (start 136.525 69.72) (end 140.335 69.72) (width 0.6) (layer "B.Cu") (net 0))
 (segment (start 142.5 90.805) (end 142.5 95.25) (width 0.6) (layer "B.Cu") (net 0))
 (segment (start 149.86 97.285) (end 149.61 97.285) (width 0.3) (layer "B.Cu") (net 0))
 (segment (start 151.384 81.534) (end 154.305 84.455) (width 0.6) (layer "B.Cu") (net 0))
 (segment (start 137.16 73.155) (end 136.525 72.52) (width 0.6) (layer "B.Cu") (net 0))
 (segment (start 137.16 81.915) (end 133.985 85.09) (width 0.6) (layer "B.Cu") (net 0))
 (segment (start 131.195 82.175) (end 131.445 82.175) (width 0.6) (layer "B.Cu") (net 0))
 (segment (start 123.19 98.795) (end 123.19 97.92) (width 0.25) (layer "B.Cu") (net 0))
 (segment (start 131.445 79.375) (end 128.905 79.375) (width 0.6) (layer "B.Cu") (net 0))
 (segment (start 138.475 90.805) (end 137.16 92.12) (width 0.6) (layer "B.Cu") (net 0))
 (segment (start 120.015 73.66) (end 120.015 66.675) (width 0.6) (layer "B.Cu") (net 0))
 (segment (start 123.317 101.092) (end 122.555 100.33) (width 0.25) (layer "B.Cu") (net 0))
 (segment (start 128.27 66.04) (end 142.24 66.04) (width 1) (layer "B.Cu") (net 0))
 (segment (start 128.27 85.09) (end 128.27 83.82) (width 0.6) (layer "B.Cu") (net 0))
 (segment (start 149.225 97.285) (end 150.495 97.285) (width 0.6) (layer "B.Cu") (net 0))
 (segment (start 133.35 95.25) (end 134.62 93.98) (width 0.6) (layer "B.Cu") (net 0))
 (segment (start 139.7 76.2) (end 139.7 73.155) (width 0.6) (layer "B.Cu") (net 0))
 (segment (start 145.803 101.092) (end 145.415 101.092) (width 0.3) (layer "B.Cu") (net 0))
 (segment (start 142.5 95.5) (end 142.5 95.25) (width 0.6) (layer "B.Cu") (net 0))
 (segment (start 120.015 91.44) (end 120.015 88.9) (width 1) (layer "B.Cu") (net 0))
 (segment (start 147.955 74.295) (end 147.955 81.915) (width 0.6) (layer "B.Cu") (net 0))
 (segment (start 143.595 86.36) (end 146.05 88.815) (width 0.6) (layer "B.Cu") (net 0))
 (segment (start 130.81 95.25) (end 133.35 95.25) (width 0.6) (layer "B.Cu") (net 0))
 (segment (start 121.666 71.273051) (end 126.899051 66.04) (width 1) (layer "B.Cu") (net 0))
 (segment (start 127 76.2) (end 127 71.501) (width 0.6) (layer "B.Cu") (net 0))
 (segment (start 142.37 81.915) (end 143.51 81.915) (width 0.6) (layer "B.Cu") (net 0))
 (segment (start 137.16 98.070051) (end 137.16 99.06) (width 0.6) (layer "B.Cu") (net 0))
 (segment (start 139.7 73.155) (end 140.335 72.52) (width 0.6) (layer "B.Cu") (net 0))
 (segment (start 124.46 86.36) (end 124.46 91.44) (width 1) (layer "B.Cu") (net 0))
 (segment (start 127 90.17) (end 128.27 88.9) (width 0.6) (layer "B.Cu") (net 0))
 (segment (start 120.015 93.98) (end 122.05 93.98) (width 0.6) (layer "B.Cu") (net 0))
 (segment (start 127 80.01) (end 127.635 79.375) (width 0.6) (layer "B.Cu") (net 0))
 (segment (start 120.015 83.82) (end 122.555 81.28) (width 0.6) (layer "B.Cu") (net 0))
 (segment (start 137.16 99.06) (end 137.16 99.06) (width 0.3) (layer "B.Cu") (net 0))
 (segment (start 154.305 84.455) (end 154.94 84.455) (width 0.6) (layer "B.Cu") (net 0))
 (segment (start 149.225 98.425) (end 149.225 97.285) (width 0.25) (layer "B.Cu") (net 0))
 (segment (start 149.225 86.36) (end 151.13 88.265) (width 0.6) (layer "B.Cu") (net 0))
 (segment (start 134.62 93.98) (end 134.62 88.9) (width 0.6) (layer "B.Cu") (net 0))
 (segment (start 144.78 99.06) (end 144.78 99.06) (width 0.3) (layer "B.Cu") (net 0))
 (segment (start 149.86 97.285) (end 150.495 97.285) (width 0.6) (layer "B.Cu") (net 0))
 (segment (start 144.78 97.78) (end 142.5 95.5) (width 0.6) (layer "B.Cu") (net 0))
 (segment (start 148.59 87.63) (end 148.59 93.98) (width 0.6) (layer "B.Cu") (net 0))
 (segment (start 131.445 91.7) (end 130.55 91.7) (width 0.6) (layer "B.Cu") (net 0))
 (segment (start 124.46 91.44) (end 124.46 92.71) (width 1) (layer "B.Cu") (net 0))
 (segment (start 151.384 80.394) (end 151.384 81.534) (width 0.6) (layer "B.Cu") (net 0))
 (segment (start 144.78 97.79) (end 144.78 97.78) (width 0.6) (layer "B.Cu") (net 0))
 (segment (start 121.666 72.263) (end 121.666 71.273051) (width 1) (layer "B.Cu") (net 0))
 (segment (start 130.55 91.7) (end 128.27 93.98) (width 0.6) (layer "B.Cu") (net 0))
 (segment (start 146.685 82.55) (end 147.955 83.82) (width 0.6) (layer "B.Cu") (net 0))
 (segment (start 143.51 100.33) (end 124.725 100.33) (width 0.25) (layer "B.Cu") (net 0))
 (segment (start 120.015 66.675) (end 121.92 64.77) (width 0.6) (layer "B.Cu") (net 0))
 (segment (start 124.46 82.55) (end 124.46 86.36) (width 1) (layer "B.Cu") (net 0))
 (segment (start 122.555 76.2) (end 120.015 73.66) (width 0.6) (layer "B.Cu") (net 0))
 (segment (start 145.803 101.092) (end 146.558 101.092) (width 0.25) (layer "B.Cu") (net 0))
 (segment (start 145.415 101.092) (end 123.317 101.092) (width 0.25) (layer "B.Cu") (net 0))
 (segment (start 140.335 69.72) (end 142.745 69.72) (width 0.6) (layer "B.Cu") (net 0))
 (segment (start 127.635 79.375) (end 128.905 79.375) (width 0.6) (layer "B.Cu") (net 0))
 (segment (start 128.27 93.98) (end 128.27 95.885) (width 0.6) (layer "B.Cu") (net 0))
 (segment (start 150.495 97.285) (end 152.27 97.285) (width 0.6) (layer "B.Cu") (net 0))
 (segment (start 144.78 99.06) (end 144.78 97.79) (width 0.6) (layer "B.Cu") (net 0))
 (segment (start 124.725 100.33) (end 123.19 98.795) (width 0.25) (layer "B.Cu") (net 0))
 (segment (start 148.085 94.485) (end 149.225 94.485) (width 0.6) (layer "B.Cu") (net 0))
 (segment (start 137.16 76.2) (end 137.16 73.155) (width 0.6) (layer "B.Cu") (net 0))
 (segment (start 120.015 86.36) (end 120.015 88.9) (width 1) (layer "B.Cu") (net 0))
 (segment (start 122.555 81.28) (end 122.555 76.2) (width 0.6) (layer "B.Cu") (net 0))
 (segment (start 137.16 86.36) (end 139.57 86.36) (width 0.6) (layer "B.Cu") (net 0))
 (segment (start 137.16 92.12) (end 137.16 98.070051) (width 0.6) (layer "B.Cu") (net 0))
 (segment (start 146.05 88.815) (end 146.05 92.71) (width 0.6) (layer "B.Cu") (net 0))
 (segment (start 149.225 83.185) (end 149.225 86.36) (width 0.6) (layer "B.Cu") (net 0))
 (segment (start 142.745 69.72) (end 143.51 70.485) (width 0.6) (layer "B.Cu") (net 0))
 (segment (start 126.899051 66.04) (end 128.27 66.04) (width 1) (layer "B.Cu") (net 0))
 (segment (start 143.51 70.485) (end 143.51 71.755) (width 0.6) (layer "B.Cu") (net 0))
 (segment (start 128.27 88.9) (end 129.54 88.9) (width 0.6) (layer "B.Cu") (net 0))
 (segment (start 129.915 82.175) (end 131.445 82.175) (width 0.6) (layer "B.Cu") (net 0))
 (segment (start 144.78 71.12) (end 147.955 74.295) (width 0.6) (layer "B.Cu") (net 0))
 (segment (start 128.27 83.82) (end 129.915 82.175) (width 0.6) (layer "B.Cu") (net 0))
 (segment (start 144.78 97.79) (end 148.085 94.485) (width 0.6) (layer "B.Cu") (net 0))
 (segment (start 147.955 83.82) (end 147.955 86.995) (width 0.6) (layer "B.Cu") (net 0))
 (segment (start 144.78 68.58) (end 144.78 71.12) (width 0.6) (layer "B.Cu") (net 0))
 (segment (start 122.05 93.98) (end 123.19 95.12) (width 0.6) (layer "B.Cu") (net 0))
 (segment (start 146.685 74.93) (end 146.685 82.55) (width 0.6) (layer "B.Cu") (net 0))
 (segment (start 144.78 99.06) (end 143.51 100.33) (width 0.25) (layer "B.Cu") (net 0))
 (segment (start 151.13 88.265) (end 153.67 88.265) (width 0.6) (layer "B.Cu") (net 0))
 (segment (start 149.095 94.485) (end 149.225 94.485) (width 0.6) (layer "B.Cu") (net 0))
 (segment (start 147.955 86.995) (end 148.59 87.63) (width 0.6) (layer "B.Cu") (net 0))
 (segment (start 143.51 71.755) (end 146.685 74.93) (width 0.6) (layer "B.Cu") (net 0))
 (segment (start 134.62 88.9) (end 137.16 86.36) (width 0.6) (layer "B.Cu") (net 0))
 (segment (start 130.81 85.09) (end 133.985 85.09) (width 0.6) (layer "B.Cu") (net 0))
 (segment (start 127 92.71) (end 124.46 92.71) (width 1) (layer "B.Cu") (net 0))
 (segment (start 153.413 75.565) (end 151.384 77.594) (width 0.6) (layer "B.Cu") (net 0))
 (segment (start 152.27 97.285) (end 153.67 95.885) (width 0.6) (layer "B.Cu") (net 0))
 (segment (start 142.24 66.04) (end 144.78 68.58) (width 0.6) (layer "B.Cu") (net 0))
 (segment (start 139.57 81.915) (end 137.16 81.915) (width 0.6) (layer "B.Cu") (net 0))
 (segment (start 120.015 86.36) (end 124.46 86.36) (width 1) (layer "B.Cu") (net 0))
 (segment (start 139.7 90.805) (end 138.475 90.805) (width 0.6) (layer "B.Cu") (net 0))
 (segment (start 124.46 75.057) (end 124.46 82.55) (width 1) (layer "B.Cu") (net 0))
 (segment (start 127 82.55) (end 124.46 82.55) (width 1) (layer "B.Cu") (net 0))
 (segment (start 148.59 93.98) (end 149.095 94.485) (width 0.6) (layer "B.Cu") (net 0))
 (segment (start 129.54 97.155) (end 130.175 97.155) (width 0.6) (layer "B.Cu") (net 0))
 (segment (start 130.175 97.155) (end 132.08 99.06) (width 0.6) (layer "B.Cu") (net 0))
 (segment (start 123.19 97.92) (end 121.415 97.92) (width 0.6) (layer "B.Cu") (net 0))
 (segment (start 129.54 71.501) (end 129.54 76.2) (width 0.6) (layer "B.Cu") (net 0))
 (segment (start 143.51 81.915) (end 146.05 84.455) (width 0.6) (layer "B.Cu") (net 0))
 (segment (start 145.803 101.092) (end 145.923 101.092) (width 0.25) (layer "B.Cu") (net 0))
 (segment (start 131.445 82.175) (end 131.185 82.175) (width 0.6) (layer "B.Cu") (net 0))
 (segment (start 131.445 88.9) (end 129.54 88.9) (width 0.6) (layer "B.Cu") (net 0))
 (segment (start 142.37 86.36) (end 143.595 86.36) (width 0.6) (layer "B.Cu") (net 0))
 (segment (start 146.558 101.092) (end 149.225 98.425) (width 0.25) (layer "B.Cu") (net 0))
 (segment (start 128.27 95.885) (end 129.54 97.155) (width 0.6) (layer "B.Cu") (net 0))
 (segment (start 131.445 91.7) (end 131.185 91.7) (width 0.6) (layer "B.Cu") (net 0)))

